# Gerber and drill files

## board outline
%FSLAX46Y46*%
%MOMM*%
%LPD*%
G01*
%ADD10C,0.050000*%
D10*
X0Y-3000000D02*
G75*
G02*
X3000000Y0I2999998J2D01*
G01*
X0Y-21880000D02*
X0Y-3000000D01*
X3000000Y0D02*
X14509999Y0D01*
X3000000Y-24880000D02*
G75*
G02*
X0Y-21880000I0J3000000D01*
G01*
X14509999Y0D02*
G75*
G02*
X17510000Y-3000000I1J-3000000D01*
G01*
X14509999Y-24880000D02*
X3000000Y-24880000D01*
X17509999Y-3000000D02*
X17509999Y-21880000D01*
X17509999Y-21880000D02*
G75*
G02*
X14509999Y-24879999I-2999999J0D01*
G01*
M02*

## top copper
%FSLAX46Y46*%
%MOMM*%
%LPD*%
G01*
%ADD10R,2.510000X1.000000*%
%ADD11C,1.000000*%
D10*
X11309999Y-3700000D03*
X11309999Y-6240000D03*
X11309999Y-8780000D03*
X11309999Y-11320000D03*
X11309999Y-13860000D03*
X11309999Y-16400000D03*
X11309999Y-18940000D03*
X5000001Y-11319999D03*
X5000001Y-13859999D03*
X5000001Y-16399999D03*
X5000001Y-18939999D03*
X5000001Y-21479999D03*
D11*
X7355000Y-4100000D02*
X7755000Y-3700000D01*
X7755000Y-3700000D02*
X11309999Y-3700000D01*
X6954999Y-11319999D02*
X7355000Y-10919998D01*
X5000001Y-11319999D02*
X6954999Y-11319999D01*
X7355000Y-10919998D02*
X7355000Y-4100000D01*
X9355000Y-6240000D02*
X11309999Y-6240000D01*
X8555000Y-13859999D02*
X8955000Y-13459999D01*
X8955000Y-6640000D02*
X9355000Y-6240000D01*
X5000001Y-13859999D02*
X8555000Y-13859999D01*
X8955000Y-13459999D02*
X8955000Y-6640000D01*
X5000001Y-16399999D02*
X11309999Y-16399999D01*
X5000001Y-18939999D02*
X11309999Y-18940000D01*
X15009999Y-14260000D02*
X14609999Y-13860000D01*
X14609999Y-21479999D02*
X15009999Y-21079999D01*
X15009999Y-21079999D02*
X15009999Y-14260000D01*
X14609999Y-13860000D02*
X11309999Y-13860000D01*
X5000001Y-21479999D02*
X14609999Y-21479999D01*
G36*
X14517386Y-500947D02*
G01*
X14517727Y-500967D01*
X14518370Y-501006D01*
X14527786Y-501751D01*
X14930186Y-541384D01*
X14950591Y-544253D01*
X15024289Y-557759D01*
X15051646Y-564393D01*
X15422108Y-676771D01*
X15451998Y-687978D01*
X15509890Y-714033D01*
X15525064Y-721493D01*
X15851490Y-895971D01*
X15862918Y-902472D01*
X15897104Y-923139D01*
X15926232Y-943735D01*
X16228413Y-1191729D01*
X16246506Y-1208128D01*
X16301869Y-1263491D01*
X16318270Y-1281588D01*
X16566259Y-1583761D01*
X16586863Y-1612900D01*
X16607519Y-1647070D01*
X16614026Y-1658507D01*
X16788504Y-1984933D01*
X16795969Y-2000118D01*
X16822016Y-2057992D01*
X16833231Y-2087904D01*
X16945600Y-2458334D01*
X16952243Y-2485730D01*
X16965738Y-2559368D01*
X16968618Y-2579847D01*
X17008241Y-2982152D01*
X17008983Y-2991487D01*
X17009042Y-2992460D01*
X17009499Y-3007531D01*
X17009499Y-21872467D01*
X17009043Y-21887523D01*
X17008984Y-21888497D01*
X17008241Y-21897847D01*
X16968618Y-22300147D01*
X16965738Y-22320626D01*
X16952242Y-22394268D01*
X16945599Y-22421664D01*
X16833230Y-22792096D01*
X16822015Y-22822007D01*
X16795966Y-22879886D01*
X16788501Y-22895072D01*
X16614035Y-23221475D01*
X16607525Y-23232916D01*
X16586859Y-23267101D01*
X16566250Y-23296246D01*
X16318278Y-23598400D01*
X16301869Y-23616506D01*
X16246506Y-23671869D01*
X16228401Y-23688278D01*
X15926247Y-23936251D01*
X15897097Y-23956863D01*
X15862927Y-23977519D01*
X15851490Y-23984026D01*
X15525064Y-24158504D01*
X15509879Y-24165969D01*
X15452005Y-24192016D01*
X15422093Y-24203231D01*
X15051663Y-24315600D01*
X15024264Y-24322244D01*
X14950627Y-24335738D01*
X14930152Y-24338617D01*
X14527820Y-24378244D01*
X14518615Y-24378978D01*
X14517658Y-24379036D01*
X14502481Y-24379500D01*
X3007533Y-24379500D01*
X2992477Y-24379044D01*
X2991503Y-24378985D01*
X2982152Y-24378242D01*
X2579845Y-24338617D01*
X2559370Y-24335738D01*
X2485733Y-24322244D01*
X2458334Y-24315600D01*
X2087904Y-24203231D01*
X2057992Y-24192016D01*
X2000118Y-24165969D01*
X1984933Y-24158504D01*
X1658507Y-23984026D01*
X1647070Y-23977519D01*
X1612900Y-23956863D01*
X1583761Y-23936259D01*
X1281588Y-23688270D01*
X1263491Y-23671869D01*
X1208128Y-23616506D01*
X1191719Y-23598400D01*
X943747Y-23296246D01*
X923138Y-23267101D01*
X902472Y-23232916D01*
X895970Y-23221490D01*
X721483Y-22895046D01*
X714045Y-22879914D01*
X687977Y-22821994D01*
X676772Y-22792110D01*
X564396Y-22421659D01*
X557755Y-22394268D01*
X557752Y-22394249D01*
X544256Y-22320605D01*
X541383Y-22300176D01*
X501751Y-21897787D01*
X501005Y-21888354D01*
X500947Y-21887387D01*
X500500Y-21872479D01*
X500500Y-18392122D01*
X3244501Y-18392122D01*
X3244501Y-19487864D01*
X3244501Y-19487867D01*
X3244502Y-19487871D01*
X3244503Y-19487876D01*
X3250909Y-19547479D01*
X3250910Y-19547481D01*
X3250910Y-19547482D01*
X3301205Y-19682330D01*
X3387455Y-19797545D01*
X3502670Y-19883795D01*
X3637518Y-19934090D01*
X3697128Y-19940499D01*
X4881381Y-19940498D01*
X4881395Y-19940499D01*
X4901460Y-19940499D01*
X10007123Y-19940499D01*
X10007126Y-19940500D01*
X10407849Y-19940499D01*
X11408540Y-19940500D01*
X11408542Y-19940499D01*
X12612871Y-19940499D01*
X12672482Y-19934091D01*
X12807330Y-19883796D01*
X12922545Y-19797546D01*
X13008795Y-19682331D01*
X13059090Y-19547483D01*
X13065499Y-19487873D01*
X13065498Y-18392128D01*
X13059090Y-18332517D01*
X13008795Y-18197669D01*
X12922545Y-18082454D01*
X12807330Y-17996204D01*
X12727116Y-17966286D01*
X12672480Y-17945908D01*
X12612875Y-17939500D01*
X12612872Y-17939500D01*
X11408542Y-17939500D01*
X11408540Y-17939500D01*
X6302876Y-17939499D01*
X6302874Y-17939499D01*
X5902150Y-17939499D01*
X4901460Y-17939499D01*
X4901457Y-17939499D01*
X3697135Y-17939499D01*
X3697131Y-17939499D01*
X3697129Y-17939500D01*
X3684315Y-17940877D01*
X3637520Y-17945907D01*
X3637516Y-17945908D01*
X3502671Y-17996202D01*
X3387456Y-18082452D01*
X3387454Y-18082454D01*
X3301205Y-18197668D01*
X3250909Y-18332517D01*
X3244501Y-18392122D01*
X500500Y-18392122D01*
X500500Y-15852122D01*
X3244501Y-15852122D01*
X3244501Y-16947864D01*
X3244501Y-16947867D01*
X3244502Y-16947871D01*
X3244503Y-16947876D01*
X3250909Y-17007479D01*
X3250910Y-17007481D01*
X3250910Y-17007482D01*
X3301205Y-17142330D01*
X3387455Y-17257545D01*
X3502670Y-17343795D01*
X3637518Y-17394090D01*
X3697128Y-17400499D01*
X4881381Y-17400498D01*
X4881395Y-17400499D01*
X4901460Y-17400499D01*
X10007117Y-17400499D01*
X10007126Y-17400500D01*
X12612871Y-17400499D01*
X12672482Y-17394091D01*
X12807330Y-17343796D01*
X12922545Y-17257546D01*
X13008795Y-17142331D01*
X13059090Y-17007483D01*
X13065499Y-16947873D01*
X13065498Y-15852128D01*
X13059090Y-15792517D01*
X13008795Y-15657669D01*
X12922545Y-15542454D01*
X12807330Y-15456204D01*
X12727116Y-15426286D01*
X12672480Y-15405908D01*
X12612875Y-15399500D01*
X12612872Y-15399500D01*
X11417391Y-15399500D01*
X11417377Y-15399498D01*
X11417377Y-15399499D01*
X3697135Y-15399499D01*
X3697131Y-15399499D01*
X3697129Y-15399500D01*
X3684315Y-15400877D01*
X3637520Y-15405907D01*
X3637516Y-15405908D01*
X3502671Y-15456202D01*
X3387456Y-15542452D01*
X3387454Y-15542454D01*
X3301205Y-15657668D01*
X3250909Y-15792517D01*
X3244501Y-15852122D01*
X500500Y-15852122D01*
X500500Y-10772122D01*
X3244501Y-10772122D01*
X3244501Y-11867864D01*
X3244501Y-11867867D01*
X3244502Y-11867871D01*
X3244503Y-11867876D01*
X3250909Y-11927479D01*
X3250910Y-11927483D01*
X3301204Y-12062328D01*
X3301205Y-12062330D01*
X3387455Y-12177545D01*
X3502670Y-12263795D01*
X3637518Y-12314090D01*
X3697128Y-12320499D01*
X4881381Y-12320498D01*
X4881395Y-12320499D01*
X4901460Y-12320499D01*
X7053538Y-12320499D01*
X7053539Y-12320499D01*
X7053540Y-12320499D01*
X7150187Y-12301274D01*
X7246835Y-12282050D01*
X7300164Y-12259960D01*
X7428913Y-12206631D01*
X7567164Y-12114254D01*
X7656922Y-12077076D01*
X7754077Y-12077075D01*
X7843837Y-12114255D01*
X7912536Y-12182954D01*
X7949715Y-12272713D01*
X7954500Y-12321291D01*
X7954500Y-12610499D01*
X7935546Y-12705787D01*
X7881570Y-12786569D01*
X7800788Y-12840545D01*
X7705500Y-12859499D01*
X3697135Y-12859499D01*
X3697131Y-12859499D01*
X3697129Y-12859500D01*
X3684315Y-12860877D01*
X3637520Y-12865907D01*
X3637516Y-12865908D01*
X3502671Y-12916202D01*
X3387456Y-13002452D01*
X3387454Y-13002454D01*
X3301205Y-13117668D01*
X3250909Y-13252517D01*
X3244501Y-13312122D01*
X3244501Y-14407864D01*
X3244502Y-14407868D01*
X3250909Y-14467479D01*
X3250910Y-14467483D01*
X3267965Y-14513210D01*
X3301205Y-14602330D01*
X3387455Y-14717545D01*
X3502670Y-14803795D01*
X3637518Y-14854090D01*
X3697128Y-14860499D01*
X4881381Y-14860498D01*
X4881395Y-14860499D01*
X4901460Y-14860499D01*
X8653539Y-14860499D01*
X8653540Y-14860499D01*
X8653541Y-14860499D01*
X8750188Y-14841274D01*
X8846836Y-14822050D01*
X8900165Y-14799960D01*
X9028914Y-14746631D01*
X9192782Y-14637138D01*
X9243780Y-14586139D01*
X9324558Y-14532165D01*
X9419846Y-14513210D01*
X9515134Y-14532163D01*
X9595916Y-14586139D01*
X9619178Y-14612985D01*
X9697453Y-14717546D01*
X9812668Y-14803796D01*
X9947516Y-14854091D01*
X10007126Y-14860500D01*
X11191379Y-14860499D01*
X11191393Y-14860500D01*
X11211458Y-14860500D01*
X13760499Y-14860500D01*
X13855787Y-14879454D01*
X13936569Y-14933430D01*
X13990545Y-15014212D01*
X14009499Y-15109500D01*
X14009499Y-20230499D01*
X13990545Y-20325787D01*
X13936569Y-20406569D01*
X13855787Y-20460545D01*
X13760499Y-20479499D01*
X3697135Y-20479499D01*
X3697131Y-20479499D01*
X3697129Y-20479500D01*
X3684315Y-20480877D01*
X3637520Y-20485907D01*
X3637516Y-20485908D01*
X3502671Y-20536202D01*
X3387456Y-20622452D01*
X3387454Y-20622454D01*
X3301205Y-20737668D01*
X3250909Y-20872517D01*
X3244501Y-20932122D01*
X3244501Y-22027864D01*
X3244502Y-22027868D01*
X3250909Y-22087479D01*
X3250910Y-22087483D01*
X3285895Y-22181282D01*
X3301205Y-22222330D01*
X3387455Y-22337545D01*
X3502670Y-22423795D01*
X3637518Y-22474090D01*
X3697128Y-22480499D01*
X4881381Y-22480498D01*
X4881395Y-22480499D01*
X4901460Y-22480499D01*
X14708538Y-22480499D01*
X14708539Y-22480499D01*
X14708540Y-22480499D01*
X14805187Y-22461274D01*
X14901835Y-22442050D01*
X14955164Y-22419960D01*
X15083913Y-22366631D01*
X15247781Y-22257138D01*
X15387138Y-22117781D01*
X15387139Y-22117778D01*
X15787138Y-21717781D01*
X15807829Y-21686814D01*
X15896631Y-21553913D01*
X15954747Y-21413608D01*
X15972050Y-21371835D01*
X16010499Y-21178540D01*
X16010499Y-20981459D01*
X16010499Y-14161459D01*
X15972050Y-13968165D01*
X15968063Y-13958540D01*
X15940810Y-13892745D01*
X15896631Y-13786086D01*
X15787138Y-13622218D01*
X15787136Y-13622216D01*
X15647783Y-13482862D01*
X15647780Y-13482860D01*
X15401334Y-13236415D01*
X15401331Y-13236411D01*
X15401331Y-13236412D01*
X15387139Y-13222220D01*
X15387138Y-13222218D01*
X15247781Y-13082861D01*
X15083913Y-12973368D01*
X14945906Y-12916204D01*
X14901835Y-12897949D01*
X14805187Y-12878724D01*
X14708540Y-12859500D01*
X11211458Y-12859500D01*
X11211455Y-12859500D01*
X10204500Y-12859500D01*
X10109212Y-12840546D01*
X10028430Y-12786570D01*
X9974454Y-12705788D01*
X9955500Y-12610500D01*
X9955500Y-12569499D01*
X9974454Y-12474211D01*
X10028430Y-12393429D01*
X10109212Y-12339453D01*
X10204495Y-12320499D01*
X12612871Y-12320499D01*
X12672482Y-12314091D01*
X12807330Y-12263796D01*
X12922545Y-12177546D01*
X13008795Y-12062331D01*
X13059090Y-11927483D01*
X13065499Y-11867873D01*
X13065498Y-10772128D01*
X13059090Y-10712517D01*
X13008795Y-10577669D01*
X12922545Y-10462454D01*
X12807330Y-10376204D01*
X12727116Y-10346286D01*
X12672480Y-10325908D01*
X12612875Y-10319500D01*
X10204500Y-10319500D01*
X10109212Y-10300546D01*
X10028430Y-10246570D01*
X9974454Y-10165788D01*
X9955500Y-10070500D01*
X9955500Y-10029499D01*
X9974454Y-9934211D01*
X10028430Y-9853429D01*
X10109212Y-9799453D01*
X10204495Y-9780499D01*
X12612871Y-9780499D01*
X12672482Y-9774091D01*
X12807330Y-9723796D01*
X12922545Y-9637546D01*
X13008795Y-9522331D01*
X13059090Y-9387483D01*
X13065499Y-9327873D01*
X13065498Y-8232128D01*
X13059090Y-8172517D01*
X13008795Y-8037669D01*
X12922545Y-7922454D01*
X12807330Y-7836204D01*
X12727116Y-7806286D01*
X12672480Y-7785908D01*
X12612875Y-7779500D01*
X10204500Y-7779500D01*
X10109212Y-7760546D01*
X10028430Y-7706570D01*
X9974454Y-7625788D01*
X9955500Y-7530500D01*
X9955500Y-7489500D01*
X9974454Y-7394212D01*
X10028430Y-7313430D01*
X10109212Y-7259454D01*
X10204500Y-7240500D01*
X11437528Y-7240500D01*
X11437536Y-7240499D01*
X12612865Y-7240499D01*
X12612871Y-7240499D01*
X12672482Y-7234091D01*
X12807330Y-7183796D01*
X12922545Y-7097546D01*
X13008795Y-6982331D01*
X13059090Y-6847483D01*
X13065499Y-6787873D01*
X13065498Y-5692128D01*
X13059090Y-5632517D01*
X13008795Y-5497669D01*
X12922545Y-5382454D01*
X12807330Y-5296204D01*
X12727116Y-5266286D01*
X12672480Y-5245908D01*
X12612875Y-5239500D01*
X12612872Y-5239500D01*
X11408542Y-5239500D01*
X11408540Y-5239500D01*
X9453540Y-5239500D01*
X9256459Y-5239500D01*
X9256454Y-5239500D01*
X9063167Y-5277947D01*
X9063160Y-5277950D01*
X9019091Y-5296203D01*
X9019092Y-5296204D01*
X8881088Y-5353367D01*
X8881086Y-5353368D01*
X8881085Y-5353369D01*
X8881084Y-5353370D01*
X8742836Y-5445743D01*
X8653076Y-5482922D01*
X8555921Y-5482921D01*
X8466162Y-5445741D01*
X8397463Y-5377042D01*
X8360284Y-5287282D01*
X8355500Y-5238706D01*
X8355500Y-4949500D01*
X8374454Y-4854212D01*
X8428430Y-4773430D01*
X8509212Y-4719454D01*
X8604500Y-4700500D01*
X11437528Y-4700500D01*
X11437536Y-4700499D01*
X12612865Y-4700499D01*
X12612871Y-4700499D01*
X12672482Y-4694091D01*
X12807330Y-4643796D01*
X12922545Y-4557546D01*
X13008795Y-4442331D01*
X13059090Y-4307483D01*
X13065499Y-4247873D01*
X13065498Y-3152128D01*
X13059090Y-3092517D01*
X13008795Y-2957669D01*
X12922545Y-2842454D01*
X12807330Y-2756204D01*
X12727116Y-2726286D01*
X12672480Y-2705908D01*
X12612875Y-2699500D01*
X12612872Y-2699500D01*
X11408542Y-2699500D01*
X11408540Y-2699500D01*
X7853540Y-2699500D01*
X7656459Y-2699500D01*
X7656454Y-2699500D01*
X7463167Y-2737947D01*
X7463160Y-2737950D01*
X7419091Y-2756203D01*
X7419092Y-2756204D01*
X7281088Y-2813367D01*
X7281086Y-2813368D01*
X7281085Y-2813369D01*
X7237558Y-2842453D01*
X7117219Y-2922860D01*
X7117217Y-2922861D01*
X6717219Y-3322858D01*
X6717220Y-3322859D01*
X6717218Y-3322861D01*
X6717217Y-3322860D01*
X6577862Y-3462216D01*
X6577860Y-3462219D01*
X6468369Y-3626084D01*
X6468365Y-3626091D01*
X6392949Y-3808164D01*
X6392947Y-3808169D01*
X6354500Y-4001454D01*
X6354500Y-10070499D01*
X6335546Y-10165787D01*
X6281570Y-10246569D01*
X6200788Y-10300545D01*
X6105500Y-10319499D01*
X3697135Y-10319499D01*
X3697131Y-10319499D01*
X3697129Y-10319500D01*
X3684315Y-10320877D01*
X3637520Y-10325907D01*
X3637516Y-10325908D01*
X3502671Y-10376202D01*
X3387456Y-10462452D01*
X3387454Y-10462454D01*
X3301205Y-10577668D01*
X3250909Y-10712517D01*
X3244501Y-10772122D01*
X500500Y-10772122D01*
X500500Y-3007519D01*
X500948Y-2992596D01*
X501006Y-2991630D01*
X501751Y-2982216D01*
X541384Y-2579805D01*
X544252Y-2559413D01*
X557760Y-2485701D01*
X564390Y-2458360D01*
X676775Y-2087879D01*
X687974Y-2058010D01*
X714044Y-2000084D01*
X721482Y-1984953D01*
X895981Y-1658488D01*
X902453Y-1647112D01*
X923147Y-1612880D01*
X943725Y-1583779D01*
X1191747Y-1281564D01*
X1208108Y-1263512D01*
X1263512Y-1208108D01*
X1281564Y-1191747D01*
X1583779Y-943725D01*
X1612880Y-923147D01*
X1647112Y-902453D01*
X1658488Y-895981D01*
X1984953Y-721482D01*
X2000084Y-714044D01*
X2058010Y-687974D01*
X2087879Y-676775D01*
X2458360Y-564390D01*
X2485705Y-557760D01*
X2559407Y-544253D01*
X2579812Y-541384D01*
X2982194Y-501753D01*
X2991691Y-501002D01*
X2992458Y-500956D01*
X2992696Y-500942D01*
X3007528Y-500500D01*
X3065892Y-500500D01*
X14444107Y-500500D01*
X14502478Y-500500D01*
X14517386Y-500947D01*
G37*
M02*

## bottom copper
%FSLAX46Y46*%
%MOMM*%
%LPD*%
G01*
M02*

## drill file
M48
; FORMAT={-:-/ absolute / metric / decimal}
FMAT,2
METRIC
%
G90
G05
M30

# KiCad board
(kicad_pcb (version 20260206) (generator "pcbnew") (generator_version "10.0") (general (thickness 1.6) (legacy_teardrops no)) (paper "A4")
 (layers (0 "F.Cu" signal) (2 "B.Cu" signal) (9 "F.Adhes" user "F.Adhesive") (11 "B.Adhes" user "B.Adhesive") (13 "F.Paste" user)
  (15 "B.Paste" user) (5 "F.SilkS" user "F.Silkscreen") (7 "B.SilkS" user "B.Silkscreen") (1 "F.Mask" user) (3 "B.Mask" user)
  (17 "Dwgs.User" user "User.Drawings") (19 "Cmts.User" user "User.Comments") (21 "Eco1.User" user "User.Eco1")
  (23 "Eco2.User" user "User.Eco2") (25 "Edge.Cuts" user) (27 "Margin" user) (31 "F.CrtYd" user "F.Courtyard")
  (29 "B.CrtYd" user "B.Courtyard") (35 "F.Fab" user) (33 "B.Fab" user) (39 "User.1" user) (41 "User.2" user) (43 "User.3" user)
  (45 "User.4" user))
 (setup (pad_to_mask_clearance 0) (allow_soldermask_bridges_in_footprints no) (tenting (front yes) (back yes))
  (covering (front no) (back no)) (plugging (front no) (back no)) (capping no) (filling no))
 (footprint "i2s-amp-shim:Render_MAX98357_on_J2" (layer "F.Cu") (at 18.009999 11.32)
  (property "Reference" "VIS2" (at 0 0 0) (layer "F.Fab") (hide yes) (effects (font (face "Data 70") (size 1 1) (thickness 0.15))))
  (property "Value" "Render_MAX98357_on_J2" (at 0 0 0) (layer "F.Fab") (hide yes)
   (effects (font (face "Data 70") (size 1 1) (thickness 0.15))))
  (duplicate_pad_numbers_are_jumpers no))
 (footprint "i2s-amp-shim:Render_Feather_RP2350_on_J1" (layer "F.Cu") (at -1.699999 16.399999)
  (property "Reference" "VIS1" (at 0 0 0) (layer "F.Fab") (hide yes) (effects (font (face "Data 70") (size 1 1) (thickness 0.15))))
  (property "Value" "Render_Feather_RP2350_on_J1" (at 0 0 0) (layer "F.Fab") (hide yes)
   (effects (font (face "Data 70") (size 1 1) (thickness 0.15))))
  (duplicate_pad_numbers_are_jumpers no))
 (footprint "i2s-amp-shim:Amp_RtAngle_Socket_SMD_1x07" (layer "F.Cu") (at 18.009999 11.32)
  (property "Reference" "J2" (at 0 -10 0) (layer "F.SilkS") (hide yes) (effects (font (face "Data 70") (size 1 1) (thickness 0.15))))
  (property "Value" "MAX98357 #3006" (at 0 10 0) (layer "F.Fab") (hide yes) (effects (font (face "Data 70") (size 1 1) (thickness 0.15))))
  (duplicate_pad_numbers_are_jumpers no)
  (pad "1" smd rect (at -6.7 -7.62) (size 2.51 1) (layers "F.Cu" "F.Mask" "F.Paste") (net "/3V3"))
  (pad "2" smd rect (at -6.7 -5.08) (size 2.51 1) (layers "F.Cu" "F.Mask" "F.Paste") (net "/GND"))
  (pad "3" smd rect (at -6.7 -2.54) (size 2.51 1) (layers "F.Cu" "F.Mask" "F.Paste") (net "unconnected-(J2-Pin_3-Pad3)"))
  (pad "4" smd rect (at -6.7 0) (size 2.51 1) (layers "F.Cu" "F.Mask" "F.Paste") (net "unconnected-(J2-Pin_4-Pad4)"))
  (pad "5" smd rect (at -6.7 2.54) (size 2.51 1) (layers "F.Cu" "F.Mask" "F.Paste") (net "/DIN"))
  (pad "6" smd rect (at -6.7 5.08) (size 2.51 1) (layers "F.Cu" "F.Mask" "F.Paste") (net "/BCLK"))
  (pad "7" smd rect (at -6.7 7.62) (size 2.51 1) (layers "F.Cu" "F.Mask" "F.Paste") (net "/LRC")))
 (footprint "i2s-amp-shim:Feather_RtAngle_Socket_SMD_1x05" (layer "F.Cu") (at -1.699999 16.399999)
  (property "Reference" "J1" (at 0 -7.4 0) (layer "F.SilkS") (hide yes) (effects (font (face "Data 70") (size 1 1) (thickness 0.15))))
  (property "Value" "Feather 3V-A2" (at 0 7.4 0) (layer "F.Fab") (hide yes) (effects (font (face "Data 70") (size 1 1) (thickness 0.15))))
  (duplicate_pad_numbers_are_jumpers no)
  (pad "1" smd rect (at 6.7 -5.08) (size 2.51 1) (layers "F.Cu" "F.Mask" "F.Paste") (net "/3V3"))
  (pad "2" smd rect (at 6.7 -2.54) (size 2.51 1) (layers "F.Cu" "F.Mask" "F.Paste") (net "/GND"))
  (pad "3" smd rect (at 6.7 0) (size 2.51 1) (layers "F.Cu" "F.Mask" "F.Paste") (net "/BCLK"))
  (pad "4" smd rect (at 6.7 2.54) (size 2.51 1) (layers "F.Cu" "F.Mask" "F.Paste") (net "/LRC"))
  (pad "5" smd rect (at 6.7 5.08) (size 2.51 1) (layers "F.Cu" "F.Mask" "F.Paste") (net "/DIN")))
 (gr_arc (start 0 3) (mid 0.878679 0.878679) (end 3 0) (stroke (width 0.05) (type default)) (layer "Edge.Cuts"))
 (gr_line (start 0 21.88) (end 0 3) (stroke (width 0.05) (type default)) (layer "Edge.Cuts"))
 (gr_line (start 3 0) (end 14.509999 0) (stroke (width 0.05) (type default)) (layer "Edge.Cuts"))
 (gr_arc (start 3 24.88) (mid 0.878679 24.00132) (end 0 21.88) (stroke (width 0.05) (type default)) (layer "Edge.Cuts"))
 (gr_arc (start 14.509999 0) (mid 16.63132 0.878679) (end 17.509999 3) (stroke (width 0.05) (type default)) (layer "Edge.Cuts"))
 (gr_line (start 14.509999 24.88) (end 3 24.88) (stroke (width 0.05) (type default)) (layer "Edge.Cuts"))
 (gr_line (start 17.509999 3) (end 17.509999 21.88) (stroke (width 0.05) (type default)) (layer "Edge.Cuts"))
 (gr_arc (start 17.509999 21.88) (mid 16.63132 24.00132) (end 14.509999 24.88) (stroke (width 0.05) (type default)) (layer "Edge.Cuts"))
 (segment (start 7.355 4.1) (end 7.755 3.7) (width 1) (layer "F.Cu") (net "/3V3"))
 (segment (start 7.755 3.7) (end 11.309999 3.7) (width 1) (layer "F.Cu") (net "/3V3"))
 (segment (start 6.954999 11.319999) (end 7.355 10.919998) (width 1) (layer "F.Cu") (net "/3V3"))
 (segment (start 5.000001 11.319999) (end 6.954999 11.319999) (width 1) (layer "F.Cu") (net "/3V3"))
 (segment (start 7.355 10.919998) (end 7.355 4.1) (width 1) (layer "F.Cu") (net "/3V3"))
 (segment (start 9.355 6.24) (end 11.309999 6.24) (width 1) (layer "F.Cu") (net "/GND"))
 (segment (start 8.555 13.859999) (end 8.955 13.459999) (width 1) (layer "F.Cu") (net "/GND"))
 (segment (start 8.955 6.64) (end 9.355 6.24) (width 1) (layer "F.Cu") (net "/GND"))
 (segment (start 5.000001 13.859999) (end 8.555 13.859999) (width 1) (layer "F.Cu") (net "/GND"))
 (segment (start 8.955 13.459999) (end 8.955 6.64) (width 1) (layer "F.Cu") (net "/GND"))
 (segment (start 5.000001 16.399999) (end 11.309999 16.399999) (width 1) (layer "F.Cu") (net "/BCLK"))
 (segment (start 5.000001 18.939999) (end 11.309999 18.94) (width 1) (layer "F.Cu") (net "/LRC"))
 (segment (start 15.009999 14.26) (end 14.609999 13.86) (width 1) (layer "F.Cu") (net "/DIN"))
 (segment (start 14.609999 21.479999) (end 15.009999 21.079999) (width 1) (layer "F.Cu") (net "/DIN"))
 (segment (start 15.009999 21.079999) (end 15.009999 14.26) (width 1) (layer "F.Cu") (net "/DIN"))
 (segment (start 14.609999 13.86) (end 11.309999 13.86) (width 1) (layer "F.Cu") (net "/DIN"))
 (segment (start 5.000001 21.479999) (end 14.609999 21.479999) (width 1) (layer "F.Cu") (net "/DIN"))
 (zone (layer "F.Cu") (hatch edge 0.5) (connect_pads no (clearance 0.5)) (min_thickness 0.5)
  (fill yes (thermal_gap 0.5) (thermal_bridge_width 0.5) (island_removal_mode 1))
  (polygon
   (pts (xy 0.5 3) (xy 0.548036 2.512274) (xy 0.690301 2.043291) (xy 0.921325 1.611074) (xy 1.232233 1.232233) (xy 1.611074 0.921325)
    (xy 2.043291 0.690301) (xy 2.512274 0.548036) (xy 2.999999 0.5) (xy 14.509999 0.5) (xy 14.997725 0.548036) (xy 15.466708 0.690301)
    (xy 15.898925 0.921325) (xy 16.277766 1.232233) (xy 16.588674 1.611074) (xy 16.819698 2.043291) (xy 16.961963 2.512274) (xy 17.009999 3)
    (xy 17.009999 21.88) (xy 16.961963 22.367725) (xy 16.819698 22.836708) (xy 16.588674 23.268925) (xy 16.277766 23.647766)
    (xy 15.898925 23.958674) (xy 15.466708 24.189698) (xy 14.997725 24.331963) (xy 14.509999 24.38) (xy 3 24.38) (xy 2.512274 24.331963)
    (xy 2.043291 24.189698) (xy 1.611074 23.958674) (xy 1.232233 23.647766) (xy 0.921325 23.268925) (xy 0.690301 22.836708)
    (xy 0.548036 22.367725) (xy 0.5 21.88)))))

